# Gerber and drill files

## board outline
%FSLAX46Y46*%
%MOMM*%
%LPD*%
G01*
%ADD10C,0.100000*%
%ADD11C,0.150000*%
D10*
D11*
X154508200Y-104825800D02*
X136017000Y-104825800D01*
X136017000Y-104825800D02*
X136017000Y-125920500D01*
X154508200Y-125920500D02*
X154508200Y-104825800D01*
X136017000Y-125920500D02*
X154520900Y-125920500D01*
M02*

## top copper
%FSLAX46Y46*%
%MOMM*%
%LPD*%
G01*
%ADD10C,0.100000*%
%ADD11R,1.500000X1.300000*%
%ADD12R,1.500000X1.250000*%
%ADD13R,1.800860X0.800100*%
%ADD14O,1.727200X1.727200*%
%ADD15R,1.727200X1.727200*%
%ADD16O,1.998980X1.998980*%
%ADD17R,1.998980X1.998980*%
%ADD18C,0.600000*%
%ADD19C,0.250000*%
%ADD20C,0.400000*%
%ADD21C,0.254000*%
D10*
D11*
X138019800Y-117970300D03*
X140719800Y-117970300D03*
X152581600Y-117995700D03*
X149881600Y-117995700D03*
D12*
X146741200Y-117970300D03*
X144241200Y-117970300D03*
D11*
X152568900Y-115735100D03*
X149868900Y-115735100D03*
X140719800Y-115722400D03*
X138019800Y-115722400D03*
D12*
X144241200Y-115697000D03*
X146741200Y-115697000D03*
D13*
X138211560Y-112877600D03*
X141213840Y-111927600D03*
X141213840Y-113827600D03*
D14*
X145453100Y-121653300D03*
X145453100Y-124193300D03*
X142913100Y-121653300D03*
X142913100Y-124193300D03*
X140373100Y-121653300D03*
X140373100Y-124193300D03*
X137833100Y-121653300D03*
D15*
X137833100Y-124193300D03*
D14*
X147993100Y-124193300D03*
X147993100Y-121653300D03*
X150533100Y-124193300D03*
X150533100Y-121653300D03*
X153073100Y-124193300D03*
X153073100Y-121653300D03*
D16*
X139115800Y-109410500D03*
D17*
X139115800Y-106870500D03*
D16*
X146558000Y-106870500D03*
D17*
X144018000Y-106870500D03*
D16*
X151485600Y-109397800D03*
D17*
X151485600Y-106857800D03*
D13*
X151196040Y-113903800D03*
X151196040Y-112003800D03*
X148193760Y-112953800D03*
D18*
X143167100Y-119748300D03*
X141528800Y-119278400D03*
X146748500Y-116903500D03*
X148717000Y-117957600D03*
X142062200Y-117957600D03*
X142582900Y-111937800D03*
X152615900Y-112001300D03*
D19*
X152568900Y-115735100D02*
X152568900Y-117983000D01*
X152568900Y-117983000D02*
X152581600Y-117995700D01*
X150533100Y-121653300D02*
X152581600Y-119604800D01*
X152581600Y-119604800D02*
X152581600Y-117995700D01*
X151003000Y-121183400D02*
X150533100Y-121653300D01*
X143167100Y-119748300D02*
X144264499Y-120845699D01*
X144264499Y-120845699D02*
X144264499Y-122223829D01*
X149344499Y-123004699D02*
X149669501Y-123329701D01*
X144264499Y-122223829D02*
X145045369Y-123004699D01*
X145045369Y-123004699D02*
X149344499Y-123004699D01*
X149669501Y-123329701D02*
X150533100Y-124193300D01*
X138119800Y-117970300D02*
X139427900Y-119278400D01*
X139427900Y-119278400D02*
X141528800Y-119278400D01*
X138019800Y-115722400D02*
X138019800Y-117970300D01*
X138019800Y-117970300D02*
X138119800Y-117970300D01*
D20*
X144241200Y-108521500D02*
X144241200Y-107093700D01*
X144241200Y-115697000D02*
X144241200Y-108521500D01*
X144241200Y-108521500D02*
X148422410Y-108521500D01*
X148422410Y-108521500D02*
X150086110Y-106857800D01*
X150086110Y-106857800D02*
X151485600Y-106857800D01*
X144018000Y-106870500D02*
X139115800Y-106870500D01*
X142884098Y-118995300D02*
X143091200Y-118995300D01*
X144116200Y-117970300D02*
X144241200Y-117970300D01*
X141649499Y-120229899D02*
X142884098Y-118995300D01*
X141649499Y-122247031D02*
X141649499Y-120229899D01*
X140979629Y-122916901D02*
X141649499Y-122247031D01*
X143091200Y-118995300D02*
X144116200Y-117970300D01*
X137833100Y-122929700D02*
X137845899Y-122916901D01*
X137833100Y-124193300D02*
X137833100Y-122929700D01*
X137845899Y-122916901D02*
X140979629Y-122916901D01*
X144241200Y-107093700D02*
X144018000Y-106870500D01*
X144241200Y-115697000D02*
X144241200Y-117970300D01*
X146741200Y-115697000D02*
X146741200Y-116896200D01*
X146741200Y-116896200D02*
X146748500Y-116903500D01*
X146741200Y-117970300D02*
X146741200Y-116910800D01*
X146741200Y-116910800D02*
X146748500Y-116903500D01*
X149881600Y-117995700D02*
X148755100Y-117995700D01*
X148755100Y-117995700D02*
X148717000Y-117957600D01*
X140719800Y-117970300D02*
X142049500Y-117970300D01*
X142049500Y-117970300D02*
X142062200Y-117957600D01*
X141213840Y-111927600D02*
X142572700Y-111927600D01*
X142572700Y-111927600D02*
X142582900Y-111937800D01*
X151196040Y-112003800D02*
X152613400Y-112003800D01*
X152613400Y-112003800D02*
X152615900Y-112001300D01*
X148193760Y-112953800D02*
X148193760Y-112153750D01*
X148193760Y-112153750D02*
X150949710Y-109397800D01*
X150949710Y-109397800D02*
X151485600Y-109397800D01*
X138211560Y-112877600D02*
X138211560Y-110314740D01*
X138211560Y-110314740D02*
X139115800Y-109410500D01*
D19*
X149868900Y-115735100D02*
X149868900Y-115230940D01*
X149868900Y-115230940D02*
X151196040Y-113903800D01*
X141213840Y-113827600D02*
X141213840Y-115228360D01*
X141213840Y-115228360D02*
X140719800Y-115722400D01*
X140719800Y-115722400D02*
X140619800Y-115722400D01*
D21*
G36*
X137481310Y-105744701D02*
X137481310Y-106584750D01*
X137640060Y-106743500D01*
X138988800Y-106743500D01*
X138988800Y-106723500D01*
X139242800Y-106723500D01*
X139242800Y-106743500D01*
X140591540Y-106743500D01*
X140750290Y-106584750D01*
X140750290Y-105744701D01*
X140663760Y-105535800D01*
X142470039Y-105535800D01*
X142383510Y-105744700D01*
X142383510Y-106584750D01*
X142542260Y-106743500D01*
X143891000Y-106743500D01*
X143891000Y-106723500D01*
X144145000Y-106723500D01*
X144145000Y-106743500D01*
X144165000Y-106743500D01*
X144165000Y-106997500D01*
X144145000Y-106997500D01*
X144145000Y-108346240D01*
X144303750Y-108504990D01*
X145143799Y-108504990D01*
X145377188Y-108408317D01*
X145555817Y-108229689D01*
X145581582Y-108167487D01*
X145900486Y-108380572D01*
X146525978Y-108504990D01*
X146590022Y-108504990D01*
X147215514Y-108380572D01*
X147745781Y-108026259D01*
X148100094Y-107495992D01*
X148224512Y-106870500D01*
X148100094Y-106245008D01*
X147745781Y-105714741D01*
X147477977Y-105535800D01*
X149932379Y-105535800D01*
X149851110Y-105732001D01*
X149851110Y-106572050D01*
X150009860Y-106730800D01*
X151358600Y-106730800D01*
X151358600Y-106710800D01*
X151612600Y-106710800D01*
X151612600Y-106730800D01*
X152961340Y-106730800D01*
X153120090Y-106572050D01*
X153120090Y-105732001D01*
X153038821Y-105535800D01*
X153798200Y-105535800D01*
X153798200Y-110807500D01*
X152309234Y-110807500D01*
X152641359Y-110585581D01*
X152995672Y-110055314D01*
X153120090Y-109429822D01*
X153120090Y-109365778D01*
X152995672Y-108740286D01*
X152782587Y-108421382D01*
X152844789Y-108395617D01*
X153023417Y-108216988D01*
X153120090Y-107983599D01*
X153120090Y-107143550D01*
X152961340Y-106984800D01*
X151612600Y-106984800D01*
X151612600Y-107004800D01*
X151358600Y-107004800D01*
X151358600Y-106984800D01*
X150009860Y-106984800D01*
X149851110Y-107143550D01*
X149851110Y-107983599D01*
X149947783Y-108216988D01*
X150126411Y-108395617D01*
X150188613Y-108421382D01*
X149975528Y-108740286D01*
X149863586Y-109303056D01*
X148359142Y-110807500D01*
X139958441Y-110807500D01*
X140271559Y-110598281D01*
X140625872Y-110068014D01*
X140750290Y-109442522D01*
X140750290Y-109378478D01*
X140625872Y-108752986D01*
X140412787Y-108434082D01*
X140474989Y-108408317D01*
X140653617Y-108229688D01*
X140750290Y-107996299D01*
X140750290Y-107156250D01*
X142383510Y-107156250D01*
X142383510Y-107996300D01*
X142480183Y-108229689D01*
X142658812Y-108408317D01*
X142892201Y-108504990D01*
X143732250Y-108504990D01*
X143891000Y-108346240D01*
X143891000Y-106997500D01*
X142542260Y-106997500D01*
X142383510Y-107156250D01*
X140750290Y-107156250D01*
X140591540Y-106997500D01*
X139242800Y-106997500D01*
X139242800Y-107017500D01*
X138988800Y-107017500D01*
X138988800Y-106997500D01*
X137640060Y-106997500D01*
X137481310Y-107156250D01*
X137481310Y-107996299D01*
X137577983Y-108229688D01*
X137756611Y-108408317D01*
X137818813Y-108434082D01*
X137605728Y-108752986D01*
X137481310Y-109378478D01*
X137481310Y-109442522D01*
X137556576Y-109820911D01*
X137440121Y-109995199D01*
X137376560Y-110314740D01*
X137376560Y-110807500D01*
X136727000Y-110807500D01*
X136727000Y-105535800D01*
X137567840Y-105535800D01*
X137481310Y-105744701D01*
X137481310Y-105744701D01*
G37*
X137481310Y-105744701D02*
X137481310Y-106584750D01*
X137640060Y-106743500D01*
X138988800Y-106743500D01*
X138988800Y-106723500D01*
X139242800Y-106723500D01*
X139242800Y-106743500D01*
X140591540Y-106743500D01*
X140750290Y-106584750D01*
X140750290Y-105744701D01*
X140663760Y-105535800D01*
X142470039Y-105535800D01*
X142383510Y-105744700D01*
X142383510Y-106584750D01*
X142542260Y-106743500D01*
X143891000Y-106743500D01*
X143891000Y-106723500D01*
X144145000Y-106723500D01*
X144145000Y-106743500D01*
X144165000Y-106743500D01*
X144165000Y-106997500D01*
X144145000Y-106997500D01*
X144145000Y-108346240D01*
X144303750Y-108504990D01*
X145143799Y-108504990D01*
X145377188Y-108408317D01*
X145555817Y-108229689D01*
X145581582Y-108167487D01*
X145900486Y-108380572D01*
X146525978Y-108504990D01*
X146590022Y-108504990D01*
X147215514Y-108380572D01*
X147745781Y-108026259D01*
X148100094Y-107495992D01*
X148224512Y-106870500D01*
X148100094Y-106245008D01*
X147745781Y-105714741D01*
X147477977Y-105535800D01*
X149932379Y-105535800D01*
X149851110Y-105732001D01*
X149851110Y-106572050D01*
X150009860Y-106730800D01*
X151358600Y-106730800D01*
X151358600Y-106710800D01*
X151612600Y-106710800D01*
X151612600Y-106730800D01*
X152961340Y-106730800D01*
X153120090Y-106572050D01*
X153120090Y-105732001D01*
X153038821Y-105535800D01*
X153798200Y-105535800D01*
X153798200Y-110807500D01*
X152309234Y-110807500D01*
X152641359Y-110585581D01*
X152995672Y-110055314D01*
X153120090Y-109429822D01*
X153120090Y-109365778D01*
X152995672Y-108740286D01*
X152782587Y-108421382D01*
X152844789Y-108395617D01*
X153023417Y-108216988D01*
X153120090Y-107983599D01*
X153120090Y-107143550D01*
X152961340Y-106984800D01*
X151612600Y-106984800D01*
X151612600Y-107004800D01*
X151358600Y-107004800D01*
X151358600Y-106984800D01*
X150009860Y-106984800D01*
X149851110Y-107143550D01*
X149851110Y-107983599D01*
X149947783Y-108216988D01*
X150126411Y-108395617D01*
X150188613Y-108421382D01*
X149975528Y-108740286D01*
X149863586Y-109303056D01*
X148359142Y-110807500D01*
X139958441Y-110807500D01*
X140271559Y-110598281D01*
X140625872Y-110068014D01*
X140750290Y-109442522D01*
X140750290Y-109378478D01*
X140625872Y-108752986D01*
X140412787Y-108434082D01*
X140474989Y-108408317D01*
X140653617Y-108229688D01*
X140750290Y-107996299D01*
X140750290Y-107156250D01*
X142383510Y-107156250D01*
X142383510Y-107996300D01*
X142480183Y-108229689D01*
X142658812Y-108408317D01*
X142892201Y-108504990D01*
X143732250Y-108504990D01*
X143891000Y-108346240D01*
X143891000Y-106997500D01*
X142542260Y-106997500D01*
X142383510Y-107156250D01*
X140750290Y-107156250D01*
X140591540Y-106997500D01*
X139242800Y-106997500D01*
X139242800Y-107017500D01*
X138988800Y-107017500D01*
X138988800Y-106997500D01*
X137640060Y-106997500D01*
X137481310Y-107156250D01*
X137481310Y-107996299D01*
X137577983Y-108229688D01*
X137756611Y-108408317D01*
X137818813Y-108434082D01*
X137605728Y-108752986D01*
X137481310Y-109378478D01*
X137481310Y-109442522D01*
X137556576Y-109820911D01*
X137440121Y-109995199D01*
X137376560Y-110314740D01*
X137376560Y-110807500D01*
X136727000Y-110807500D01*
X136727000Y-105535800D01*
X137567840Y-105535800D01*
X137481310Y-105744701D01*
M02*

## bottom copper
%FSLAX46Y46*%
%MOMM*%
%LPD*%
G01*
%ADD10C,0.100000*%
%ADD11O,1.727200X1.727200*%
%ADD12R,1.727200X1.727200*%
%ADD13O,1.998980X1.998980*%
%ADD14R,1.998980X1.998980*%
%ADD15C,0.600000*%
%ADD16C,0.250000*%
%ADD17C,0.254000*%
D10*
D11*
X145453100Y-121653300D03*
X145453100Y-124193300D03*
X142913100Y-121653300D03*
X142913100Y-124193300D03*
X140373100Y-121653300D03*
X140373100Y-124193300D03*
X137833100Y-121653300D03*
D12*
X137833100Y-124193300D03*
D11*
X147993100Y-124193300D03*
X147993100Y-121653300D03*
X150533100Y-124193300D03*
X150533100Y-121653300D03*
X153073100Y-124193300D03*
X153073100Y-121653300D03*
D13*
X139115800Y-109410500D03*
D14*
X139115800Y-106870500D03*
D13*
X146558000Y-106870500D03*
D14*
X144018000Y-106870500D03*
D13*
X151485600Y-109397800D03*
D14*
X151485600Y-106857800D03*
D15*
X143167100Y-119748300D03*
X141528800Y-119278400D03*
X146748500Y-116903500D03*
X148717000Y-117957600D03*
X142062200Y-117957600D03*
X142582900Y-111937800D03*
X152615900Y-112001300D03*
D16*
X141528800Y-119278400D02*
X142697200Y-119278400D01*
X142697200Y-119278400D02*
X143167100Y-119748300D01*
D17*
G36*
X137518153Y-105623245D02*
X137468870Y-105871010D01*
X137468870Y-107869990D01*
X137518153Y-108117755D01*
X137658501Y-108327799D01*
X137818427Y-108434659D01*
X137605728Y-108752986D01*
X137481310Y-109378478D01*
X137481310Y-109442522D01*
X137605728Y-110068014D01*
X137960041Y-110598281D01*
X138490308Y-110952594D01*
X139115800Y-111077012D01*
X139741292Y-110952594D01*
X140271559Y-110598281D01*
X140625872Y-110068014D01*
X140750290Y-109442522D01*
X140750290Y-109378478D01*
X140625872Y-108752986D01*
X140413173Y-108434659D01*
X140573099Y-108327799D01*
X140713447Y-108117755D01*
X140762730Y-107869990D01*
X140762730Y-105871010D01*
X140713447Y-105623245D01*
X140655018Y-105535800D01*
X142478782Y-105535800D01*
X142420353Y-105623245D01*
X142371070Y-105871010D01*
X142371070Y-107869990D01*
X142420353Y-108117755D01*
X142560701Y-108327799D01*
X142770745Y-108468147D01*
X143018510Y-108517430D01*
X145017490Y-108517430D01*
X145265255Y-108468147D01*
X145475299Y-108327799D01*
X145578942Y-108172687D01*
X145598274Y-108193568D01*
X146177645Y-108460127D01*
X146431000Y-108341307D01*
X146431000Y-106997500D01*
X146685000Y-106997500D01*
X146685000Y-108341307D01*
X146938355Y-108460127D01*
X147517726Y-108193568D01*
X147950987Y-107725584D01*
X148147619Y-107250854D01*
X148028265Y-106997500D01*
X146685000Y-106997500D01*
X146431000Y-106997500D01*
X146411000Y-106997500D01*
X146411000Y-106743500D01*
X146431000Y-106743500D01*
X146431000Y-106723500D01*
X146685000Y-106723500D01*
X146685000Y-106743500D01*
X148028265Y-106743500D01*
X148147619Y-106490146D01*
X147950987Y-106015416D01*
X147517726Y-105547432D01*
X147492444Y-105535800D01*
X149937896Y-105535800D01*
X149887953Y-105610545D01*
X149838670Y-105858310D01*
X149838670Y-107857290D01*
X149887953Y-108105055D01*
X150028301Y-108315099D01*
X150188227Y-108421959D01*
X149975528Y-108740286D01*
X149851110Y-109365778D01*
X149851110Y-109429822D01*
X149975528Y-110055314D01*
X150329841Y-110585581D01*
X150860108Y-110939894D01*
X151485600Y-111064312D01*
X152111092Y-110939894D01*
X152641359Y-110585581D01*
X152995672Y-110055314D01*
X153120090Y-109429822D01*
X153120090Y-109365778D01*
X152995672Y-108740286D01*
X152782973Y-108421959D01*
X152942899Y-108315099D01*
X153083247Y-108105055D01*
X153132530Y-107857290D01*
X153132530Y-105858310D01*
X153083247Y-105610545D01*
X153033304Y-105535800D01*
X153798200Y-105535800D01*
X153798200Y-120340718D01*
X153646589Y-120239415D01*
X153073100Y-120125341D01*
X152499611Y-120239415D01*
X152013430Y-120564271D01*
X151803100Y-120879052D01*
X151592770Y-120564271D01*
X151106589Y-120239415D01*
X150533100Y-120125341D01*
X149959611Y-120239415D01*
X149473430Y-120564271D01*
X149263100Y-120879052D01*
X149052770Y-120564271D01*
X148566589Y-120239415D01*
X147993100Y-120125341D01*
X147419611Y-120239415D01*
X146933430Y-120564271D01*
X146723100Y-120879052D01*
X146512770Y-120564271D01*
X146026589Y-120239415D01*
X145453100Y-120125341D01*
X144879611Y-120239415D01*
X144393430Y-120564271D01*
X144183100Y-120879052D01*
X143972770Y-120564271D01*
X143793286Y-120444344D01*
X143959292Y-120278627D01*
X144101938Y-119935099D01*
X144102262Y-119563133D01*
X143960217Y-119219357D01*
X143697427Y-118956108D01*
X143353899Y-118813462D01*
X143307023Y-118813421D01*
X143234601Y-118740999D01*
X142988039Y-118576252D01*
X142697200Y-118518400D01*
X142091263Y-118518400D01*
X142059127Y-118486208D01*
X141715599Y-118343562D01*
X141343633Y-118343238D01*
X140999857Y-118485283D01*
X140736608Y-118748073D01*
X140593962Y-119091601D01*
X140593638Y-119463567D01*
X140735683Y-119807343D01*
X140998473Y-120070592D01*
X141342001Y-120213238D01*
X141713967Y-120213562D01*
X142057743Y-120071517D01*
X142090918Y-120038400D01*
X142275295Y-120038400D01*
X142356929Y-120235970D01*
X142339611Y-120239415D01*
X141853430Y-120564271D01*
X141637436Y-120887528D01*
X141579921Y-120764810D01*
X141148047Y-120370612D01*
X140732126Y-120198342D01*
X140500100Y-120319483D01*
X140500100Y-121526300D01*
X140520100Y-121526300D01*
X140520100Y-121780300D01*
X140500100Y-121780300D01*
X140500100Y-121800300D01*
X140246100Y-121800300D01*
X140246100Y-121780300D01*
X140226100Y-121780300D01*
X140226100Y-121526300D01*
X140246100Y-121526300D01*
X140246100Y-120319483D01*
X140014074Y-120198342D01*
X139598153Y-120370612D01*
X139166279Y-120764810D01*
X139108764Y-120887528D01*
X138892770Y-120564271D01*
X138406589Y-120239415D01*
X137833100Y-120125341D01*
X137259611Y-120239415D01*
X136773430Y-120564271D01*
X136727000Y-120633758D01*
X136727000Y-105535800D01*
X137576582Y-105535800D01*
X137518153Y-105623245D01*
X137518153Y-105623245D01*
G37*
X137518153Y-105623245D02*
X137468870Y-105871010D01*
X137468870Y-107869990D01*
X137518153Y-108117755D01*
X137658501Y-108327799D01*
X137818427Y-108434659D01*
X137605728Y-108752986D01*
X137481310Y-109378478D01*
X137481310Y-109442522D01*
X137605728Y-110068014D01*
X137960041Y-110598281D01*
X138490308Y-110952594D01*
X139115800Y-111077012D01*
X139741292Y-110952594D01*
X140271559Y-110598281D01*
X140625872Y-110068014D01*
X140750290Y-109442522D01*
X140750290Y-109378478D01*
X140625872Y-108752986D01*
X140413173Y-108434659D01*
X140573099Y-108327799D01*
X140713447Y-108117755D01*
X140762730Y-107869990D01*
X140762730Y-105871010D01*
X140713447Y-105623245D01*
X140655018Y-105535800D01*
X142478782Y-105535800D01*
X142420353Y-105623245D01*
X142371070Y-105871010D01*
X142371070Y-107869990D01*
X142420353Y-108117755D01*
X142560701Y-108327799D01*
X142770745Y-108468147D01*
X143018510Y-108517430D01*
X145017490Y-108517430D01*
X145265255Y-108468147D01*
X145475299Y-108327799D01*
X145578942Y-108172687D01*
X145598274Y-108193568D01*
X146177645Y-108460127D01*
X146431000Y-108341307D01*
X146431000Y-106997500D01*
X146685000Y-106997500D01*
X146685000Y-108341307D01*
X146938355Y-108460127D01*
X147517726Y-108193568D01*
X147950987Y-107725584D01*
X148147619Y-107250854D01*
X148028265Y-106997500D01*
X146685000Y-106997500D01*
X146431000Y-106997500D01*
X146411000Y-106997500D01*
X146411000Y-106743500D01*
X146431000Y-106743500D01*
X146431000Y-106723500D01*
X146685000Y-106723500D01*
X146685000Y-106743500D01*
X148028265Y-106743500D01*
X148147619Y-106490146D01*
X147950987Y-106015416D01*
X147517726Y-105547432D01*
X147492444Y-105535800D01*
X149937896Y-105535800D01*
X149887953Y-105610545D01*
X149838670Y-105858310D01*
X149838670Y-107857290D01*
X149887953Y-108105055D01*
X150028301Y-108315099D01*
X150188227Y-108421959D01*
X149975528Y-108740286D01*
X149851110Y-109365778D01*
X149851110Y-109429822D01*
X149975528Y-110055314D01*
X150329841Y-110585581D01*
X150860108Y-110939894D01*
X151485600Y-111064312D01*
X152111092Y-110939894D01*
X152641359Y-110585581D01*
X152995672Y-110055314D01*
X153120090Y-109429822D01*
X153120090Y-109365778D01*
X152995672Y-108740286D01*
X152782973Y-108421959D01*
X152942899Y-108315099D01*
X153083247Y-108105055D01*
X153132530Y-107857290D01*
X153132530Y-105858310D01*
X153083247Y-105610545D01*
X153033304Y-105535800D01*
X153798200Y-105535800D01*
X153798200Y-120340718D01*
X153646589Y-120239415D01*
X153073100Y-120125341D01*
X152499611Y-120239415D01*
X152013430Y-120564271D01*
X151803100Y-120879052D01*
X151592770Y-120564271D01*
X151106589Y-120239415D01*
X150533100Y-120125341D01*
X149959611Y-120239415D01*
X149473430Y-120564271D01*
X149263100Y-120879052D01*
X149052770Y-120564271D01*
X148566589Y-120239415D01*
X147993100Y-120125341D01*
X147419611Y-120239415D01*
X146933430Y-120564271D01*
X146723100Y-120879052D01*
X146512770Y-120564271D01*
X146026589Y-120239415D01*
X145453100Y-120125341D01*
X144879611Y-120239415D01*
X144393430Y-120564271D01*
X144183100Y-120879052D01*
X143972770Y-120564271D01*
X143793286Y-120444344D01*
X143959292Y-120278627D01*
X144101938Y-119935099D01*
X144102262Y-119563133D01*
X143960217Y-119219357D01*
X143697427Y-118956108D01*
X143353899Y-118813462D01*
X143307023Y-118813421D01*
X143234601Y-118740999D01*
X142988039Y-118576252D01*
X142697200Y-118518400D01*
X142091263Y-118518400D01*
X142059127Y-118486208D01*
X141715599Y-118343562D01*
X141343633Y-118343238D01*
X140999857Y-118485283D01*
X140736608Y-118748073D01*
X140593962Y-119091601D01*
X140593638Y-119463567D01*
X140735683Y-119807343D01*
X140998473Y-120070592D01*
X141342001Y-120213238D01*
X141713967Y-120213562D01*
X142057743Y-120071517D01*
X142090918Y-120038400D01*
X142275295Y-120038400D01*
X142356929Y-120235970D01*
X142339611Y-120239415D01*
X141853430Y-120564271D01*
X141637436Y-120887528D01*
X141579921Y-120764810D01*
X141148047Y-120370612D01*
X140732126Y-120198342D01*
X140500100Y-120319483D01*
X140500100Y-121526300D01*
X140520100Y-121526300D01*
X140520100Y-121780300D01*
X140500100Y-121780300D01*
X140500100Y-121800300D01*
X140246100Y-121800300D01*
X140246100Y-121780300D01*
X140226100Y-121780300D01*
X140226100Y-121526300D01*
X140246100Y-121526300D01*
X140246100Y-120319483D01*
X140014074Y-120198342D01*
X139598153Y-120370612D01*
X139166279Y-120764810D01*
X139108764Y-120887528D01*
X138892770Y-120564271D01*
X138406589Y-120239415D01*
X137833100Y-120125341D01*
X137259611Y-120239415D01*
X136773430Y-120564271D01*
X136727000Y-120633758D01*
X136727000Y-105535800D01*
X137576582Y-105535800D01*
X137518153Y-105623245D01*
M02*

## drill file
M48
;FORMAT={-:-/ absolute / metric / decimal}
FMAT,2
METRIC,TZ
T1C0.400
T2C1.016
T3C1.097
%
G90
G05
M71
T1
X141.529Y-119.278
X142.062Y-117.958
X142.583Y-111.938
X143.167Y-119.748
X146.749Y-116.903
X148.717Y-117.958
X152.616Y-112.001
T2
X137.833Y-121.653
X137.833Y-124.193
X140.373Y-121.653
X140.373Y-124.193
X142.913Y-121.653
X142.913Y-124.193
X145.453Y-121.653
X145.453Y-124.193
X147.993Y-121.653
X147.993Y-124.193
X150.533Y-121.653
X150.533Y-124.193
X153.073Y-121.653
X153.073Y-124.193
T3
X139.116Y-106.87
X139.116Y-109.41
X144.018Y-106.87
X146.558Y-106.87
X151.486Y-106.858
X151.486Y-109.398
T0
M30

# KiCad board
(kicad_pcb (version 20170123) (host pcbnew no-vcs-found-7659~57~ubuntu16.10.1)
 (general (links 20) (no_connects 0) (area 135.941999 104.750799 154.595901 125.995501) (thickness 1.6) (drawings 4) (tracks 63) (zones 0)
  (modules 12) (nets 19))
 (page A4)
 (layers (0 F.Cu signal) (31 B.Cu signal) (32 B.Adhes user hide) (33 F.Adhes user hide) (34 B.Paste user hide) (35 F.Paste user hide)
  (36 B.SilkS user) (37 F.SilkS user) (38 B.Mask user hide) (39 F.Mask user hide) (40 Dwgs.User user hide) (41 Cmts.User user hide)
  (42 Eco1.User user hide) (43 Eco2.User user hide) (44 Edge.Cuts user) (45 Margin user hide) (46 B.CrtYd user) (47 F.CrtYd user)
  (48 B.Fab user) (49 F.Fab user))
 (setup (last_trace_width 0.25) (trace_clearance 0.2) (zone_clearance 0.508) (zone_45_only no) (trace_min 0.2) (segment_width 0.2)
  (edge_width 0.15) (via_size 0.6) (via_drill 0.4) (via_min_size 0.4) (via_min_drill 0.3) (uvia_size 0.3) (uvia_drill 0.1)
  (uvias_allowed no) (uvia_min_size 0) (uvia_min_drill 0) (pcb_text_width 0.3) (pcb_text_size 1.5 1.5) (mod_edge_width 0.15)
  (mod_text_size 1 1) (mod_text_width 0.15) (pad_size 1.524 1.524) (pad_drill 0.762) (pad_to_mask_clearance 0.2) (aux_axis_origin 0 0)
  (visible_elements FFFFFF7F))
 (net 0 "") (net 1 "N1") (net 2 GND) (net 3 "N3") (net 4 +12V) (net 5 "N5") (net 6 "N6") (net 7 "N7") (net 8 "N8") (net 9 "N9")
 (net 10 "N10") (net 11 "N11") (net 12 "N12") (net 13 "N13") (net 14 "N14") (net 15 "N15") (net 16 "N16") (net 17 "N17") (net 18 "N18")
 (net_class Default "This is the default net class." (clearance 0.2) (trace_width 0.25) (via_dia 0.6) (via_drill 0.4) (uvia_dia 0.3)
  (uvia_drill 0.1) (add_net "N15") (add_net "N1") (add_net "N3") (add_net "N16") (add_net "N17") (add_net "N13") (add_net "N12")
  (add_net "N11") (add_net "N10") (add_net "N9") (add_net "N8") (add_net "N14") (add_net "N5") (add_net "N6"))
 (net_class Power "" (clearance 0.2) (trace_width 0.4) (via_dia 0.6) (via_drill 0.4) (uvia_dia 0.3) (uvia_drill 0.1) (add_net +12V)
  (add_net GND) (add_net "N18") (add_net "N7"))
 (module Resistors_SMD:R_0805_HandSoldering (layer F.Cu) (at 139.3698 117.9703)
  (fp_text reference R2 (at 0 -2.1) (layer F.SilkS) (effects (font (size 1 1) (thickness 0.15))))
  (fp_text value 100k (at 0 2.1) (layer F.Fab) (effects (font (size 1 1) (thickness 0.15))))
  (pad 1 smd rect (at -1.35 0) (size 1.5 1.3) (layers F.Cu F.Paste F.Mask) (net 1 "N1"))
  (pad 2 smd rect (at 1.35 0) (size 1.5 1.3) (layers F.Cu F.Paste F.Mask) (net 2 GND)))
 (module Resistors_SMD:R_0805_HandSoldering (layer F.Cu) (at 151.2316 117.9957 180)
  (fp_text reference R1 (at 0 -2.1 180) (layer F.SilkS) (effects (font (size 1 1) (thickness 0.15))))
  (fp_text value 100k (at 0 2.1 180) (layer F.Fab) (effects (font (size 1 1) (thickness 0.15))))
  (pad 1 smd rect (at -1.35 0 180) (size 1.5 1.3) (layers F.Cu F.Paste F.Mask) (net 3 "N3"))
  (pad 2 smd rect (at 1.35 0 180) (size 1.5 1.3) (layers F.Cu F.Paste F.Mask) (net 2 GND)))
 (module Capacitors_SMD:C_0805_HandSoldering (layer F.Cu) (at 145.4912 117.9703)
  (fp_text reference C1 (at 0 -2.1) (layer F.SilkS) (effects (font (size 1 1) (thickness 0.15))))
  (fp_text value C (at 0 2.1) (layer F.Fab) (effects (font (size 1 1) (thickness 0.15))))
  (pad 2 smd rect (at 1.25 0) (size 1.5 1.25) (layers F.Cu F.Paste F.Mask) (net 2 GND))
  (pad 1 smd rect (at -1.25 0) (size 1.5 1.25) (layers F.Cu F.Paste F.Mask) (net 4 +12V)))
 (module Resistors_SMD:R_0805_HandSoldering (layer F.Cu) (at 151.2189 115.7351)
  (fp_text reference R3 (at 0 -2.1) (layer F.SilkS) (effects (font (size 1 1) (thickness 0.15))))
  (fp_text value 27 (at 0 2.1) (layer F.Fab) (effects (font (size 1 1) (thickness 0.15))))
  (pad 2 smd rect (at 1.35 0) (size 1.5 1.3) (layers F.Cu F.Paste F.Mask) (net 3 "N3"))
  (pad 1 smd rect (at -1.35 0) (size 1.5 1.3) (layers F.Cu F.Paste F.Mask) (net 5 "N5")))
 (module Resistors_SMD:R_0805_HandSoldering (layer F.Cu) (at 139.3698 115.7224 180)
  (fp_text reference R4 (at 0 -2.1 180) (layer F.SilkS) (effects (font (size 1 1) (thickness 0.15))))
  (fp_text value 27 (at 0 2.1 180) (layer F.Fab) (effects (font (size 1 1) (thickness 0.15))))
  (pad 1 smd rect (at -1.35 0 180) (size 1.5 1.3) (layers F.Cu F.Paste F.Mask) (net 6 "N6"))
  (pad 2 smd rect (at 1.35 0 180) (size 1.5 1.3) (layers F.Cu F.Paste F.Mask) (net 1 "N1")))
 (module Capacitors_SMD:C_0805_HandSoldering (layer F.Cu) (at 145.4912 115.697)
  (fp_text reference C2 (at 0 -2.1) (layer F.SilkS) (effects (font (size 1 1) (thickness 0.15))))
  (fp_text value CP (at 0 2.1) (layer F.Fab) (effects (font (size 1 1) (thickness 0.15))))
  (pad 1 smd rect (at -1.25 0) (size 1.5 1.25) (layers F.Cu F.Paste F.Mask) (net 4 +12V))
  (pad 2 smd rect (at 1.25 0) (size 1.5 1.25) (layers F.Cu F.Paste F.Mask) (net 2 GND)))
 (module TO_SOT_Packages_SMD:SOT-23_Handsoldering (layer F.Cu) (at 139.7127 112.8776 90)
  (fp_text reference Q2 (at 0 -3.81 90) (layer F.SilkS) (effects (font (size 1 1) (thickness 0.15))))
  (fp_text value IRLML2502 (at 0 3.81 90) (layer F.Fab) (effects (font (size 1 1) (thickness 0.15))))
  (pad 3 smd rect (at 0 -1.50114 90) (size 0.8001 1.80086) (layers F.Cu F.Paste F.Mask) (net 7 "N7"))
  (pad 2 smd rect (at 0.95 1.50114 90) (size 0.8001 1.80086) (layers F.Cu F.Paste F.Mask) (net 2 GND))
  (pad 1 smd rect (at -0.95 1.50114 90) (size 0.8001 1.80086) (layers F.Cu F.Paste F.Mask) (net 6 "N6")))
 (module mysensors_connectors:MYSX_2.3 (layer F.Cu) (at 137.8331 124.1933 90)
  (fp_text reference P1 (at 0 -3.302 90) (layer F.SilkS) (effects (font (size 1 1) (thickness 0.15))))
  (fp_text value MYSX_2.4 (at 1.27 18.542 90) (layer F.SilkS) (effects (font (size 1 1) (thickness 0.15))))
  (pad 8 thru_hole oval (at 2.54 7.62 90) (size 1.7272 1.7272) (drill 1.016) (layers *.Cu *.Mask F.SilkS) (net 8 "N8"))
  (pad 7 thru_hole oval (at 0 7.62 90) (size 1.7272 1.7272) (drill 1.016) (layers *.Cu *.Mask F.SilkS) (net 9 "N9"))
  (pad 6 thru_hole oval (at 2.54 5.08 90) (size 1.7272 1.7272) (drill 1.016) (layers *.Cu *.Mask F.SilkS) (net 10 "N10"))
  (pad 5 thru_hole oval (at 0 5.08 90) (size 1.7272 1.7272) (drill 1.016) (layers *.Cu *.Mask F.SilkS) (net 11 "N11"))
  (pad 4 thru_hole oval (at 2.54 2.54 90) (size 1.7272 1.7272) (drill 1.016) (layers *.Cu *.Mask F.SilkS) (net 2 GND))
  (pad 3 thru_hole oval (at 0 2.54 90) (size 1.7272 1.7272) (drill 1.016) (layers *.Cu *.Mask F.SilkS) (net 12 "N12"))
  (pad 2 thru_hole oval (at 2.54 0 90) (size 1.7272 1.7272) (drill 1.016) (layers *.Cu *.Mask F.SilkS) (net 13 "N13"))
  (pad 1 thru_hole rect (at 0 0 90) (size 1.7272 1.7272) (drill 1.016) (layers *.Cu *.Mask F.SilkS) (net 4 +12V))
  (pad 9 thru_hole oval (at 0 10.16 90) (size 1.7272 1.7272) (drill 1.016) (layers *.Cu *.Mask F.SilkS) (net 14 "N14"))
  (pad 10 thru_hole oval (at 2.54 10.16 90) (size 1.7272 1.7272) (drill 1.016) (layers *.Cu *.Mask F.SilkS) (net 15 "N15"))
  (pad 11 thru_hole oval (at 0 12.7 90) (size 1.7272 1.7272) (drill 1.016) (layers *.Cu *.Mask F.SilkS) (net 1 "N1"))
  (pad 12 thru_hole oval (at 2.54 12.7 90) (size 1.7272 1.7272) (drill 1.016) (layers *.Cu *.Mask F.SilkS) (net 3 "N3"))
  (pad 13 thru_hole oval (at 0 15.24 90) (size 1.7272 1.7272) (drill 1.016) (layers *.Cu *.Mask F.SilkS) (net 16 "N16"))
  (pad 14 thru_hole oval (at 2.54 15.24 90) (size 1.7272 1.7272) (drill 1.016) (layers *.Cu *.Mask F.SilkS) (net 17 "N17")))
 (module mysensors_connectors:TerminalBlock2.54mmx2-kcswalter (layer F.Cu) (at 139.1158 108.1405 90)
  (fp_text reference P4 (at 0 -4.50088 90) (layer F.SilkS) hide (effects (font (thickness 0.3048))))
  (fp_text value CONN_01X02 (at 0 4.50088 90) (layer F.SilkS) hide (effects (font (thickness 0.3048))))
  (pad 2 thru_hole oval (at -1.27 0 90) (size 1.99898 1.99898) (drill 1.09728) (layers *.Cu *.Mask F.SilkS) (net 7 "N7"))
  (pad 1 thru_hole rect (at 1.27 0 90) (size 1.99898 1.99898) (drill 1.09728) (layers *.Cu *.Mask F.SilkS) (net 4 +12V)))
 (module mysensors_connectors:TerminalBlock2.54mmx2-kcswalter (layer F.Cu) (at 145.288 106.8705 180)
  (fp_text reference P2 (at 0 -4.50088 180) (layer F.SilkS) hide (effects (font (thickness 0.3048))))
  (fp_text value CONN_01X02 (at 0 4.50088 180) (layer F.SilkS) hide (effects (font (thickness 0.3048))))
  (pad 2 thru_hole oval (at -1.27 0 180) (size 1.99898 1.99898) (drill 1.09728) (layers *.Cu *.Mask F.SilkS) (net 2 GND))
  (pad 1 thru_hole rect (at 1.27 0 180) (size 1.99898 1.99898) (drill 1.09728) (layers *.Cu *.Mask F.SilkS) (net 4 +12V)))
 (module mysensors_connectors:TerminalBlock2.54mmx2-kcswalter (layer F.Cu) (at 151.4856 108.1278 90)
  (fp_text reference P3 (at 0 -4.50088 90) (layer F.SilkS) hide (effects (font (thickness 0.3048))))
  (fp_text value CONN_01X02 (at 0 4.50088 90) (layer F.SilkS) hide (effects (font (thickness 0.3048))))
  (pad 2 thru_hole oval (at -1.27 0 90) (size 1.99898 1.99898) (drill 1.09728) (layers *.Cu *.Mask F.SilkS) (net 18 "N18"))
  (pad 1 thru_hole rect (at 1.27 0 90) (size 1.99898 1.99898) (drill 1.09728) (layers *.Cu *.Mask F.SilkS) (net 4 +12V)))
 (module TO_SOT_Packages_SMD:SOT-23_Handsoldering (layer F.Cu) (at 149.6949 112.9538 90)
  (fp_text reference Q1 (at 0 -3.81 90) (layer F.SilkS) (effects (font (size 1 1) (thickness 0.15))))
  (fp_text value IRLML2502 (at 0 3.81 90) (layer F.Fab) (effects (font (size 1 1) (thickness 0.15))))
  (pad 1 smd rect (at -0.95 1.50114 90) (size 0.8001 1.80086) (layers F.Cu F.Paste F.Mask) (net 5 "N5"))
  (pad 2 smd rect (at 0.95 1.50114 90) (size 0.8001 1.80086) (layers F.Cu F.Paste F.Mask) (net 2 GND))
  (pad 3 smd rect (at 0 -1.50114 90) (size 0.8001 1.80086) (layers F.Cu F.Paste F.Mask) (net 18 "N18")))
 (gr_line (start 154.5082 104.8258) (end 136.017 104.8258) (layer Edge.Cuts) (width 0.15))
 (gr_line (start 136.017 104.8258) (end 136.017 125.9205) (layer Edge.Cuts) (width 0.15))
 (gr_line (start 154.5082 125.9205) (end 154.5082 104.8258) (layer Edge.Cuts) (width 0.15))
 (gr_line (start 136.017 125.9205) (end 154.5082 125.9205) (layer Edge.Cuts) (width 0.15))
 (segment (start 152.5689 115.7351) (end 152.5689 117.983) (width 0.25) (layer F.Cu) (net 3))
 (segment (start 152.5689 117.983) (end 152.5816 117.9957) (width 0.25) (layer F.Cu) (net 3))
 (segment (start 150.5331 121.6533) (end 152.5816 119.6048) (width 0.25) (layer F.Cu) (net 3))
 (segment (start 152.5816 119.6048) (end 152.5816 117.9957) (width 0.25) (layer F.Cu) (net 3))
 (segment (start 151.003 121.1834) (end 150.5331 121.6533) (width 0.25) (layer F.Cu) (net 3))
 (segment (start 143.1671 119.7483) (end 144.264499 120.845699) (width 0.25) (layer F.Cu) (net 1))
 (segment (start 144.264499 120.845699) (end 144.264499 122.223829) (width 0.25) (layer F.Cu) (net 1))
 (segment (start 149.344499 123.004699) (end 149.669501 123.329701) (width 0.25) (layer F.Cu) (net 1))
 (segment (start 144.264499 122.223829) (end 145.045369 123.004699) (width 0.25) (layer F.Cu) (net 1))
 (segment (start 145.045369 123.004699) (end 149.344499 123.004699) (width 0.25) (layer F.Cu) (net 1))
 (segment (start 149.669501 123.329701) (end 150.5331 124.1933) (width 0.25) (layer F.Cu) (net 1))
 (segment (start 141.5288 119.2784) (end 142.6972 119.2784) (width 0.25) (layer B.Cu) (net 1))
 (segment (start 142.6972 119.2784) (end 143.1671 119.7483) (width 0.25) (layer B.Cu) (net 1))
 (via (at 143.1671 119.7483) (size 0.6) (drill 0.4) (layers F.Cu B.Cu) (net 1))
 (segment (start 138.1198 117.9703) (end 139.4279 119.2784) (width 0.25) (layer F.Cu) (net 1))
 (segment (start 139.4279 119.2784) (end 141.5288 119.2784) (width 0.25) (layer F.Cu) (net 1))
 (via (at 141.5288 119.2784) (size 0.6) (drill 0.4) (layers F.Cu B.Cu) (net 1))
 (segment (start 138.0198 115.7224) (end 138.0198 117.9703) (width 0.25) (layer F.Cu) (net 1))
 (segment (start 138.0198 117.9703) (end 138.1198 117.9703) (width 0.25) (layer F.Cu) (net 1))
 (segment (start 144.2412 108.5215) (end 144.2412 107.0937) (width 0.4) (layer F.Cu) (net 4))
 (segment (start 144.2412 115.697) (end 144.2412 108.5215) (width 0.4) (layer F.Cu) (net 4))
 (segment (start 144.2412 108.5215) (end 148.42241 108.5215) (width 0.4) (layer F.Cu) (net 4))
 (segment (start 148.42241 108.5215) (end 150.08611 106.8578) (width 0.4) (layer F.Cu) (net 4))
 (segment (start 150.08611 106.8578) (end 151.4856 106.8578) (width 0.4) (layer F.Cu) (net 4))
 (segment (start 144.018 106.8705) (end 139.1158 106.8705) (width 0.4) (layer F.Cu) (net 4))
 (segment (start 142.884098 118.9953) (end 143.0912 118.9953) (width 0.4) (layer F.Cu) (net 4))
 (segment (start 144.1162 117.9703) (end 144.2412 117.9703) (width 0.4) (layer F.Cu) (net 4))
 (segment (start 141.649499 120.229899) (end 142.884098 118.9953) (width 0.4) (layer F.Cu) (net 4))
 (segment (start 141.649499 122.247031) (end 141.649499 120.229899) (width 0.4) (layer F.Cu) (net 4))
 (segment (start 140.979629 122.916901) (end 141.649499 122.247031) (width 0.4) (layer F.Cu) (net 4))
 (segment (start 143.0912 118.9953) (end 144.1162 117.9703) (width 0.4) (layer F.Cu) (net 4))
 (segment (start 137.8331 122.9297) (end 137.845899 122.916901) (width 0.4) (layer F.Cu) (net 4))
 (segment (start 137.8331 124.1933) (end 137.8331 122.9297) (width 0.4) (layer F.Cu) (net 4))
 (segment (start 137.845899 122.916901) (end 140.979629 122.916901) (width 0.4) (layer F.Cu) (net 4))
 (segment (start 144.2412 107.0937) (end 144.018 106.8705) (width 0.4) (layer F.Cu) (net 4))
 (segment (start 144.2412 115.697) (end 144.2412 117.9703) (width 0.4) (layer F.Cu) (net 4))
 (segment (start 146.7412 115.697) (end 146.7412 116.8962) (width 0.4) (layer F.Cu) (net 2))
 (segment (start 146.7412 116.8962) (end 146.7485 116.9035) (width 0.4) (layer F.Cu) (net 2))
 (segment (start 146.7412 117.9703) (end 146.7412 116.9108) (width 0.4) (layer F.Cu) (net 2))
 (segment (start 146.7412 116.9108) (end 146.7485 116.9035) (width 0.4) (layer F.Cu) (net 2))
 (via (at 146.7485 116.9035) (size 0.6) (drill 0.4) (layers F.Cu B.Cu) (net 2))
 (segment (start 149.8816 117.9957) (end 148.7551 117.9957) (width 0.4) (layer F.Cu) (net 2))
 (segment (start 148.7551 117.9957) (end 148.717 117.9576) (width 0.4) (layer F.Cu) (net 2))
 (via (at 148.717 117.9576) (size 0.6) (drill 0.4) (layers F.Cu B.Cu) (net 2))
 (segment (start 140.7198 117.9703) (end 142.0495 117.9703) (width 0.4) (layer F.Cu) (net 2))
 (segment (start 142.0495 117.9703) (end 142.0622 117.9576) (width 0.4) (layer F.Cu) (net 2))
 (via (at 142.0622 117.9576) (size 0.6) (drill 0.4) (layers F.Cu B.Cu) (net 2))
 (segment (start 141.21384 111.9276) (end 142.5727 111.9276) (width 0.4) (layer F.Cu) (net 2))
 (segment (start 142.5727 111.9276) (end 142.5829 111.9378) (width 0.4) (layer F.Cu) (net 2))
 (via (at 142.5829 111.9378) (size 0.6) (drill 0.4) (layers F.Cu B.Cu) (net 2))
 (segment (start 151.19604 112.0038) (end 152.6134 112.0038) (width 0.4) (layer F.Cu) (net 2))
 (segment (start 152.6134 112.0038) (end 152.6159 112.0013) (width 0.4) (layer F.Cu) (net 2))
 (via (at 152.6159 112.0013) (size 0.6) (drill 0.4) (layers F.Cu B.Cu) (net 2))
 (segment (start 148.19376 112.9538) (end 148.19376 112.15375) (width 0.4) (layer F.Cu) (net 18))
 (segment (start 148.19376 112.15375) (end 150.94971 109.3978) (width 0.4) (layer F.Cu) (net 18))
 (segment (start 150.94971 109.3978) (end 151.4856 109.3978) (width 0.4) (layer F.Cu) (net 18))
 (segment (start 138.21156 112.8776) (end 138.21156 110.31474) (width 0.4) (layer F.Cu) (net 7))
 (segment (start 138.21156 110.31474) (end 139.1158 109.4105) (width 0.4) (layer F.Cu) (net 7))
 (segment (start 149.8689 115.7351) (end 149.8689 115.23094) (width 0.25) (layer F.Cu) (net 5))
 (segment (start 149.8689 115.23094) (end 151.19604 113.9038) (width 0.25) (layer F.Cu) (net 5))
 (segment (start 141.21384 113.8276) (end 141.21384 115.22836) (width 0.25) (layer F.Cu) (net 6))
 (segment (start 141.21384 115.22836) (end 140.7198 115.7224) (width 0.25) (layer F.Cu) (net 6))
 (segment (start 140.7198 115.7224) (end 140.6198 115.7224) (width 0.25) (layer F.Cu) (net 6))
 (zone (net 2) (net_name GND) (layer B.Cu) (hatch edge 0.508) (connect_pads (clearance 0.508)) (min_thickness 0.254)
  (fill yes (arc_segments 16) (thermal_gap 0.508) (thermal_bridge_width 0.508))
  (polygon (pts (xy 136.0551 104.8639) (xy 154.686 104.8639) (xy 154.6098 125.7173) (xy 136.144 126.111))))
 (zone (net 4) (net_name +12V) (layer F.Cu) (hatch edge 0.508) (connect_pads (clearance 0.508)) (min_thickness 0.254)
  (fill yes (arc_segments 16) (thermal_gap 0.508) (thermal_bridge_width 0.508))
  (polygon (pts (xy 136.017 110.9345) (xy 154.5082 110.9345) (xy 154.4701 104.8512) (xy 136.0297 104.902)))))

